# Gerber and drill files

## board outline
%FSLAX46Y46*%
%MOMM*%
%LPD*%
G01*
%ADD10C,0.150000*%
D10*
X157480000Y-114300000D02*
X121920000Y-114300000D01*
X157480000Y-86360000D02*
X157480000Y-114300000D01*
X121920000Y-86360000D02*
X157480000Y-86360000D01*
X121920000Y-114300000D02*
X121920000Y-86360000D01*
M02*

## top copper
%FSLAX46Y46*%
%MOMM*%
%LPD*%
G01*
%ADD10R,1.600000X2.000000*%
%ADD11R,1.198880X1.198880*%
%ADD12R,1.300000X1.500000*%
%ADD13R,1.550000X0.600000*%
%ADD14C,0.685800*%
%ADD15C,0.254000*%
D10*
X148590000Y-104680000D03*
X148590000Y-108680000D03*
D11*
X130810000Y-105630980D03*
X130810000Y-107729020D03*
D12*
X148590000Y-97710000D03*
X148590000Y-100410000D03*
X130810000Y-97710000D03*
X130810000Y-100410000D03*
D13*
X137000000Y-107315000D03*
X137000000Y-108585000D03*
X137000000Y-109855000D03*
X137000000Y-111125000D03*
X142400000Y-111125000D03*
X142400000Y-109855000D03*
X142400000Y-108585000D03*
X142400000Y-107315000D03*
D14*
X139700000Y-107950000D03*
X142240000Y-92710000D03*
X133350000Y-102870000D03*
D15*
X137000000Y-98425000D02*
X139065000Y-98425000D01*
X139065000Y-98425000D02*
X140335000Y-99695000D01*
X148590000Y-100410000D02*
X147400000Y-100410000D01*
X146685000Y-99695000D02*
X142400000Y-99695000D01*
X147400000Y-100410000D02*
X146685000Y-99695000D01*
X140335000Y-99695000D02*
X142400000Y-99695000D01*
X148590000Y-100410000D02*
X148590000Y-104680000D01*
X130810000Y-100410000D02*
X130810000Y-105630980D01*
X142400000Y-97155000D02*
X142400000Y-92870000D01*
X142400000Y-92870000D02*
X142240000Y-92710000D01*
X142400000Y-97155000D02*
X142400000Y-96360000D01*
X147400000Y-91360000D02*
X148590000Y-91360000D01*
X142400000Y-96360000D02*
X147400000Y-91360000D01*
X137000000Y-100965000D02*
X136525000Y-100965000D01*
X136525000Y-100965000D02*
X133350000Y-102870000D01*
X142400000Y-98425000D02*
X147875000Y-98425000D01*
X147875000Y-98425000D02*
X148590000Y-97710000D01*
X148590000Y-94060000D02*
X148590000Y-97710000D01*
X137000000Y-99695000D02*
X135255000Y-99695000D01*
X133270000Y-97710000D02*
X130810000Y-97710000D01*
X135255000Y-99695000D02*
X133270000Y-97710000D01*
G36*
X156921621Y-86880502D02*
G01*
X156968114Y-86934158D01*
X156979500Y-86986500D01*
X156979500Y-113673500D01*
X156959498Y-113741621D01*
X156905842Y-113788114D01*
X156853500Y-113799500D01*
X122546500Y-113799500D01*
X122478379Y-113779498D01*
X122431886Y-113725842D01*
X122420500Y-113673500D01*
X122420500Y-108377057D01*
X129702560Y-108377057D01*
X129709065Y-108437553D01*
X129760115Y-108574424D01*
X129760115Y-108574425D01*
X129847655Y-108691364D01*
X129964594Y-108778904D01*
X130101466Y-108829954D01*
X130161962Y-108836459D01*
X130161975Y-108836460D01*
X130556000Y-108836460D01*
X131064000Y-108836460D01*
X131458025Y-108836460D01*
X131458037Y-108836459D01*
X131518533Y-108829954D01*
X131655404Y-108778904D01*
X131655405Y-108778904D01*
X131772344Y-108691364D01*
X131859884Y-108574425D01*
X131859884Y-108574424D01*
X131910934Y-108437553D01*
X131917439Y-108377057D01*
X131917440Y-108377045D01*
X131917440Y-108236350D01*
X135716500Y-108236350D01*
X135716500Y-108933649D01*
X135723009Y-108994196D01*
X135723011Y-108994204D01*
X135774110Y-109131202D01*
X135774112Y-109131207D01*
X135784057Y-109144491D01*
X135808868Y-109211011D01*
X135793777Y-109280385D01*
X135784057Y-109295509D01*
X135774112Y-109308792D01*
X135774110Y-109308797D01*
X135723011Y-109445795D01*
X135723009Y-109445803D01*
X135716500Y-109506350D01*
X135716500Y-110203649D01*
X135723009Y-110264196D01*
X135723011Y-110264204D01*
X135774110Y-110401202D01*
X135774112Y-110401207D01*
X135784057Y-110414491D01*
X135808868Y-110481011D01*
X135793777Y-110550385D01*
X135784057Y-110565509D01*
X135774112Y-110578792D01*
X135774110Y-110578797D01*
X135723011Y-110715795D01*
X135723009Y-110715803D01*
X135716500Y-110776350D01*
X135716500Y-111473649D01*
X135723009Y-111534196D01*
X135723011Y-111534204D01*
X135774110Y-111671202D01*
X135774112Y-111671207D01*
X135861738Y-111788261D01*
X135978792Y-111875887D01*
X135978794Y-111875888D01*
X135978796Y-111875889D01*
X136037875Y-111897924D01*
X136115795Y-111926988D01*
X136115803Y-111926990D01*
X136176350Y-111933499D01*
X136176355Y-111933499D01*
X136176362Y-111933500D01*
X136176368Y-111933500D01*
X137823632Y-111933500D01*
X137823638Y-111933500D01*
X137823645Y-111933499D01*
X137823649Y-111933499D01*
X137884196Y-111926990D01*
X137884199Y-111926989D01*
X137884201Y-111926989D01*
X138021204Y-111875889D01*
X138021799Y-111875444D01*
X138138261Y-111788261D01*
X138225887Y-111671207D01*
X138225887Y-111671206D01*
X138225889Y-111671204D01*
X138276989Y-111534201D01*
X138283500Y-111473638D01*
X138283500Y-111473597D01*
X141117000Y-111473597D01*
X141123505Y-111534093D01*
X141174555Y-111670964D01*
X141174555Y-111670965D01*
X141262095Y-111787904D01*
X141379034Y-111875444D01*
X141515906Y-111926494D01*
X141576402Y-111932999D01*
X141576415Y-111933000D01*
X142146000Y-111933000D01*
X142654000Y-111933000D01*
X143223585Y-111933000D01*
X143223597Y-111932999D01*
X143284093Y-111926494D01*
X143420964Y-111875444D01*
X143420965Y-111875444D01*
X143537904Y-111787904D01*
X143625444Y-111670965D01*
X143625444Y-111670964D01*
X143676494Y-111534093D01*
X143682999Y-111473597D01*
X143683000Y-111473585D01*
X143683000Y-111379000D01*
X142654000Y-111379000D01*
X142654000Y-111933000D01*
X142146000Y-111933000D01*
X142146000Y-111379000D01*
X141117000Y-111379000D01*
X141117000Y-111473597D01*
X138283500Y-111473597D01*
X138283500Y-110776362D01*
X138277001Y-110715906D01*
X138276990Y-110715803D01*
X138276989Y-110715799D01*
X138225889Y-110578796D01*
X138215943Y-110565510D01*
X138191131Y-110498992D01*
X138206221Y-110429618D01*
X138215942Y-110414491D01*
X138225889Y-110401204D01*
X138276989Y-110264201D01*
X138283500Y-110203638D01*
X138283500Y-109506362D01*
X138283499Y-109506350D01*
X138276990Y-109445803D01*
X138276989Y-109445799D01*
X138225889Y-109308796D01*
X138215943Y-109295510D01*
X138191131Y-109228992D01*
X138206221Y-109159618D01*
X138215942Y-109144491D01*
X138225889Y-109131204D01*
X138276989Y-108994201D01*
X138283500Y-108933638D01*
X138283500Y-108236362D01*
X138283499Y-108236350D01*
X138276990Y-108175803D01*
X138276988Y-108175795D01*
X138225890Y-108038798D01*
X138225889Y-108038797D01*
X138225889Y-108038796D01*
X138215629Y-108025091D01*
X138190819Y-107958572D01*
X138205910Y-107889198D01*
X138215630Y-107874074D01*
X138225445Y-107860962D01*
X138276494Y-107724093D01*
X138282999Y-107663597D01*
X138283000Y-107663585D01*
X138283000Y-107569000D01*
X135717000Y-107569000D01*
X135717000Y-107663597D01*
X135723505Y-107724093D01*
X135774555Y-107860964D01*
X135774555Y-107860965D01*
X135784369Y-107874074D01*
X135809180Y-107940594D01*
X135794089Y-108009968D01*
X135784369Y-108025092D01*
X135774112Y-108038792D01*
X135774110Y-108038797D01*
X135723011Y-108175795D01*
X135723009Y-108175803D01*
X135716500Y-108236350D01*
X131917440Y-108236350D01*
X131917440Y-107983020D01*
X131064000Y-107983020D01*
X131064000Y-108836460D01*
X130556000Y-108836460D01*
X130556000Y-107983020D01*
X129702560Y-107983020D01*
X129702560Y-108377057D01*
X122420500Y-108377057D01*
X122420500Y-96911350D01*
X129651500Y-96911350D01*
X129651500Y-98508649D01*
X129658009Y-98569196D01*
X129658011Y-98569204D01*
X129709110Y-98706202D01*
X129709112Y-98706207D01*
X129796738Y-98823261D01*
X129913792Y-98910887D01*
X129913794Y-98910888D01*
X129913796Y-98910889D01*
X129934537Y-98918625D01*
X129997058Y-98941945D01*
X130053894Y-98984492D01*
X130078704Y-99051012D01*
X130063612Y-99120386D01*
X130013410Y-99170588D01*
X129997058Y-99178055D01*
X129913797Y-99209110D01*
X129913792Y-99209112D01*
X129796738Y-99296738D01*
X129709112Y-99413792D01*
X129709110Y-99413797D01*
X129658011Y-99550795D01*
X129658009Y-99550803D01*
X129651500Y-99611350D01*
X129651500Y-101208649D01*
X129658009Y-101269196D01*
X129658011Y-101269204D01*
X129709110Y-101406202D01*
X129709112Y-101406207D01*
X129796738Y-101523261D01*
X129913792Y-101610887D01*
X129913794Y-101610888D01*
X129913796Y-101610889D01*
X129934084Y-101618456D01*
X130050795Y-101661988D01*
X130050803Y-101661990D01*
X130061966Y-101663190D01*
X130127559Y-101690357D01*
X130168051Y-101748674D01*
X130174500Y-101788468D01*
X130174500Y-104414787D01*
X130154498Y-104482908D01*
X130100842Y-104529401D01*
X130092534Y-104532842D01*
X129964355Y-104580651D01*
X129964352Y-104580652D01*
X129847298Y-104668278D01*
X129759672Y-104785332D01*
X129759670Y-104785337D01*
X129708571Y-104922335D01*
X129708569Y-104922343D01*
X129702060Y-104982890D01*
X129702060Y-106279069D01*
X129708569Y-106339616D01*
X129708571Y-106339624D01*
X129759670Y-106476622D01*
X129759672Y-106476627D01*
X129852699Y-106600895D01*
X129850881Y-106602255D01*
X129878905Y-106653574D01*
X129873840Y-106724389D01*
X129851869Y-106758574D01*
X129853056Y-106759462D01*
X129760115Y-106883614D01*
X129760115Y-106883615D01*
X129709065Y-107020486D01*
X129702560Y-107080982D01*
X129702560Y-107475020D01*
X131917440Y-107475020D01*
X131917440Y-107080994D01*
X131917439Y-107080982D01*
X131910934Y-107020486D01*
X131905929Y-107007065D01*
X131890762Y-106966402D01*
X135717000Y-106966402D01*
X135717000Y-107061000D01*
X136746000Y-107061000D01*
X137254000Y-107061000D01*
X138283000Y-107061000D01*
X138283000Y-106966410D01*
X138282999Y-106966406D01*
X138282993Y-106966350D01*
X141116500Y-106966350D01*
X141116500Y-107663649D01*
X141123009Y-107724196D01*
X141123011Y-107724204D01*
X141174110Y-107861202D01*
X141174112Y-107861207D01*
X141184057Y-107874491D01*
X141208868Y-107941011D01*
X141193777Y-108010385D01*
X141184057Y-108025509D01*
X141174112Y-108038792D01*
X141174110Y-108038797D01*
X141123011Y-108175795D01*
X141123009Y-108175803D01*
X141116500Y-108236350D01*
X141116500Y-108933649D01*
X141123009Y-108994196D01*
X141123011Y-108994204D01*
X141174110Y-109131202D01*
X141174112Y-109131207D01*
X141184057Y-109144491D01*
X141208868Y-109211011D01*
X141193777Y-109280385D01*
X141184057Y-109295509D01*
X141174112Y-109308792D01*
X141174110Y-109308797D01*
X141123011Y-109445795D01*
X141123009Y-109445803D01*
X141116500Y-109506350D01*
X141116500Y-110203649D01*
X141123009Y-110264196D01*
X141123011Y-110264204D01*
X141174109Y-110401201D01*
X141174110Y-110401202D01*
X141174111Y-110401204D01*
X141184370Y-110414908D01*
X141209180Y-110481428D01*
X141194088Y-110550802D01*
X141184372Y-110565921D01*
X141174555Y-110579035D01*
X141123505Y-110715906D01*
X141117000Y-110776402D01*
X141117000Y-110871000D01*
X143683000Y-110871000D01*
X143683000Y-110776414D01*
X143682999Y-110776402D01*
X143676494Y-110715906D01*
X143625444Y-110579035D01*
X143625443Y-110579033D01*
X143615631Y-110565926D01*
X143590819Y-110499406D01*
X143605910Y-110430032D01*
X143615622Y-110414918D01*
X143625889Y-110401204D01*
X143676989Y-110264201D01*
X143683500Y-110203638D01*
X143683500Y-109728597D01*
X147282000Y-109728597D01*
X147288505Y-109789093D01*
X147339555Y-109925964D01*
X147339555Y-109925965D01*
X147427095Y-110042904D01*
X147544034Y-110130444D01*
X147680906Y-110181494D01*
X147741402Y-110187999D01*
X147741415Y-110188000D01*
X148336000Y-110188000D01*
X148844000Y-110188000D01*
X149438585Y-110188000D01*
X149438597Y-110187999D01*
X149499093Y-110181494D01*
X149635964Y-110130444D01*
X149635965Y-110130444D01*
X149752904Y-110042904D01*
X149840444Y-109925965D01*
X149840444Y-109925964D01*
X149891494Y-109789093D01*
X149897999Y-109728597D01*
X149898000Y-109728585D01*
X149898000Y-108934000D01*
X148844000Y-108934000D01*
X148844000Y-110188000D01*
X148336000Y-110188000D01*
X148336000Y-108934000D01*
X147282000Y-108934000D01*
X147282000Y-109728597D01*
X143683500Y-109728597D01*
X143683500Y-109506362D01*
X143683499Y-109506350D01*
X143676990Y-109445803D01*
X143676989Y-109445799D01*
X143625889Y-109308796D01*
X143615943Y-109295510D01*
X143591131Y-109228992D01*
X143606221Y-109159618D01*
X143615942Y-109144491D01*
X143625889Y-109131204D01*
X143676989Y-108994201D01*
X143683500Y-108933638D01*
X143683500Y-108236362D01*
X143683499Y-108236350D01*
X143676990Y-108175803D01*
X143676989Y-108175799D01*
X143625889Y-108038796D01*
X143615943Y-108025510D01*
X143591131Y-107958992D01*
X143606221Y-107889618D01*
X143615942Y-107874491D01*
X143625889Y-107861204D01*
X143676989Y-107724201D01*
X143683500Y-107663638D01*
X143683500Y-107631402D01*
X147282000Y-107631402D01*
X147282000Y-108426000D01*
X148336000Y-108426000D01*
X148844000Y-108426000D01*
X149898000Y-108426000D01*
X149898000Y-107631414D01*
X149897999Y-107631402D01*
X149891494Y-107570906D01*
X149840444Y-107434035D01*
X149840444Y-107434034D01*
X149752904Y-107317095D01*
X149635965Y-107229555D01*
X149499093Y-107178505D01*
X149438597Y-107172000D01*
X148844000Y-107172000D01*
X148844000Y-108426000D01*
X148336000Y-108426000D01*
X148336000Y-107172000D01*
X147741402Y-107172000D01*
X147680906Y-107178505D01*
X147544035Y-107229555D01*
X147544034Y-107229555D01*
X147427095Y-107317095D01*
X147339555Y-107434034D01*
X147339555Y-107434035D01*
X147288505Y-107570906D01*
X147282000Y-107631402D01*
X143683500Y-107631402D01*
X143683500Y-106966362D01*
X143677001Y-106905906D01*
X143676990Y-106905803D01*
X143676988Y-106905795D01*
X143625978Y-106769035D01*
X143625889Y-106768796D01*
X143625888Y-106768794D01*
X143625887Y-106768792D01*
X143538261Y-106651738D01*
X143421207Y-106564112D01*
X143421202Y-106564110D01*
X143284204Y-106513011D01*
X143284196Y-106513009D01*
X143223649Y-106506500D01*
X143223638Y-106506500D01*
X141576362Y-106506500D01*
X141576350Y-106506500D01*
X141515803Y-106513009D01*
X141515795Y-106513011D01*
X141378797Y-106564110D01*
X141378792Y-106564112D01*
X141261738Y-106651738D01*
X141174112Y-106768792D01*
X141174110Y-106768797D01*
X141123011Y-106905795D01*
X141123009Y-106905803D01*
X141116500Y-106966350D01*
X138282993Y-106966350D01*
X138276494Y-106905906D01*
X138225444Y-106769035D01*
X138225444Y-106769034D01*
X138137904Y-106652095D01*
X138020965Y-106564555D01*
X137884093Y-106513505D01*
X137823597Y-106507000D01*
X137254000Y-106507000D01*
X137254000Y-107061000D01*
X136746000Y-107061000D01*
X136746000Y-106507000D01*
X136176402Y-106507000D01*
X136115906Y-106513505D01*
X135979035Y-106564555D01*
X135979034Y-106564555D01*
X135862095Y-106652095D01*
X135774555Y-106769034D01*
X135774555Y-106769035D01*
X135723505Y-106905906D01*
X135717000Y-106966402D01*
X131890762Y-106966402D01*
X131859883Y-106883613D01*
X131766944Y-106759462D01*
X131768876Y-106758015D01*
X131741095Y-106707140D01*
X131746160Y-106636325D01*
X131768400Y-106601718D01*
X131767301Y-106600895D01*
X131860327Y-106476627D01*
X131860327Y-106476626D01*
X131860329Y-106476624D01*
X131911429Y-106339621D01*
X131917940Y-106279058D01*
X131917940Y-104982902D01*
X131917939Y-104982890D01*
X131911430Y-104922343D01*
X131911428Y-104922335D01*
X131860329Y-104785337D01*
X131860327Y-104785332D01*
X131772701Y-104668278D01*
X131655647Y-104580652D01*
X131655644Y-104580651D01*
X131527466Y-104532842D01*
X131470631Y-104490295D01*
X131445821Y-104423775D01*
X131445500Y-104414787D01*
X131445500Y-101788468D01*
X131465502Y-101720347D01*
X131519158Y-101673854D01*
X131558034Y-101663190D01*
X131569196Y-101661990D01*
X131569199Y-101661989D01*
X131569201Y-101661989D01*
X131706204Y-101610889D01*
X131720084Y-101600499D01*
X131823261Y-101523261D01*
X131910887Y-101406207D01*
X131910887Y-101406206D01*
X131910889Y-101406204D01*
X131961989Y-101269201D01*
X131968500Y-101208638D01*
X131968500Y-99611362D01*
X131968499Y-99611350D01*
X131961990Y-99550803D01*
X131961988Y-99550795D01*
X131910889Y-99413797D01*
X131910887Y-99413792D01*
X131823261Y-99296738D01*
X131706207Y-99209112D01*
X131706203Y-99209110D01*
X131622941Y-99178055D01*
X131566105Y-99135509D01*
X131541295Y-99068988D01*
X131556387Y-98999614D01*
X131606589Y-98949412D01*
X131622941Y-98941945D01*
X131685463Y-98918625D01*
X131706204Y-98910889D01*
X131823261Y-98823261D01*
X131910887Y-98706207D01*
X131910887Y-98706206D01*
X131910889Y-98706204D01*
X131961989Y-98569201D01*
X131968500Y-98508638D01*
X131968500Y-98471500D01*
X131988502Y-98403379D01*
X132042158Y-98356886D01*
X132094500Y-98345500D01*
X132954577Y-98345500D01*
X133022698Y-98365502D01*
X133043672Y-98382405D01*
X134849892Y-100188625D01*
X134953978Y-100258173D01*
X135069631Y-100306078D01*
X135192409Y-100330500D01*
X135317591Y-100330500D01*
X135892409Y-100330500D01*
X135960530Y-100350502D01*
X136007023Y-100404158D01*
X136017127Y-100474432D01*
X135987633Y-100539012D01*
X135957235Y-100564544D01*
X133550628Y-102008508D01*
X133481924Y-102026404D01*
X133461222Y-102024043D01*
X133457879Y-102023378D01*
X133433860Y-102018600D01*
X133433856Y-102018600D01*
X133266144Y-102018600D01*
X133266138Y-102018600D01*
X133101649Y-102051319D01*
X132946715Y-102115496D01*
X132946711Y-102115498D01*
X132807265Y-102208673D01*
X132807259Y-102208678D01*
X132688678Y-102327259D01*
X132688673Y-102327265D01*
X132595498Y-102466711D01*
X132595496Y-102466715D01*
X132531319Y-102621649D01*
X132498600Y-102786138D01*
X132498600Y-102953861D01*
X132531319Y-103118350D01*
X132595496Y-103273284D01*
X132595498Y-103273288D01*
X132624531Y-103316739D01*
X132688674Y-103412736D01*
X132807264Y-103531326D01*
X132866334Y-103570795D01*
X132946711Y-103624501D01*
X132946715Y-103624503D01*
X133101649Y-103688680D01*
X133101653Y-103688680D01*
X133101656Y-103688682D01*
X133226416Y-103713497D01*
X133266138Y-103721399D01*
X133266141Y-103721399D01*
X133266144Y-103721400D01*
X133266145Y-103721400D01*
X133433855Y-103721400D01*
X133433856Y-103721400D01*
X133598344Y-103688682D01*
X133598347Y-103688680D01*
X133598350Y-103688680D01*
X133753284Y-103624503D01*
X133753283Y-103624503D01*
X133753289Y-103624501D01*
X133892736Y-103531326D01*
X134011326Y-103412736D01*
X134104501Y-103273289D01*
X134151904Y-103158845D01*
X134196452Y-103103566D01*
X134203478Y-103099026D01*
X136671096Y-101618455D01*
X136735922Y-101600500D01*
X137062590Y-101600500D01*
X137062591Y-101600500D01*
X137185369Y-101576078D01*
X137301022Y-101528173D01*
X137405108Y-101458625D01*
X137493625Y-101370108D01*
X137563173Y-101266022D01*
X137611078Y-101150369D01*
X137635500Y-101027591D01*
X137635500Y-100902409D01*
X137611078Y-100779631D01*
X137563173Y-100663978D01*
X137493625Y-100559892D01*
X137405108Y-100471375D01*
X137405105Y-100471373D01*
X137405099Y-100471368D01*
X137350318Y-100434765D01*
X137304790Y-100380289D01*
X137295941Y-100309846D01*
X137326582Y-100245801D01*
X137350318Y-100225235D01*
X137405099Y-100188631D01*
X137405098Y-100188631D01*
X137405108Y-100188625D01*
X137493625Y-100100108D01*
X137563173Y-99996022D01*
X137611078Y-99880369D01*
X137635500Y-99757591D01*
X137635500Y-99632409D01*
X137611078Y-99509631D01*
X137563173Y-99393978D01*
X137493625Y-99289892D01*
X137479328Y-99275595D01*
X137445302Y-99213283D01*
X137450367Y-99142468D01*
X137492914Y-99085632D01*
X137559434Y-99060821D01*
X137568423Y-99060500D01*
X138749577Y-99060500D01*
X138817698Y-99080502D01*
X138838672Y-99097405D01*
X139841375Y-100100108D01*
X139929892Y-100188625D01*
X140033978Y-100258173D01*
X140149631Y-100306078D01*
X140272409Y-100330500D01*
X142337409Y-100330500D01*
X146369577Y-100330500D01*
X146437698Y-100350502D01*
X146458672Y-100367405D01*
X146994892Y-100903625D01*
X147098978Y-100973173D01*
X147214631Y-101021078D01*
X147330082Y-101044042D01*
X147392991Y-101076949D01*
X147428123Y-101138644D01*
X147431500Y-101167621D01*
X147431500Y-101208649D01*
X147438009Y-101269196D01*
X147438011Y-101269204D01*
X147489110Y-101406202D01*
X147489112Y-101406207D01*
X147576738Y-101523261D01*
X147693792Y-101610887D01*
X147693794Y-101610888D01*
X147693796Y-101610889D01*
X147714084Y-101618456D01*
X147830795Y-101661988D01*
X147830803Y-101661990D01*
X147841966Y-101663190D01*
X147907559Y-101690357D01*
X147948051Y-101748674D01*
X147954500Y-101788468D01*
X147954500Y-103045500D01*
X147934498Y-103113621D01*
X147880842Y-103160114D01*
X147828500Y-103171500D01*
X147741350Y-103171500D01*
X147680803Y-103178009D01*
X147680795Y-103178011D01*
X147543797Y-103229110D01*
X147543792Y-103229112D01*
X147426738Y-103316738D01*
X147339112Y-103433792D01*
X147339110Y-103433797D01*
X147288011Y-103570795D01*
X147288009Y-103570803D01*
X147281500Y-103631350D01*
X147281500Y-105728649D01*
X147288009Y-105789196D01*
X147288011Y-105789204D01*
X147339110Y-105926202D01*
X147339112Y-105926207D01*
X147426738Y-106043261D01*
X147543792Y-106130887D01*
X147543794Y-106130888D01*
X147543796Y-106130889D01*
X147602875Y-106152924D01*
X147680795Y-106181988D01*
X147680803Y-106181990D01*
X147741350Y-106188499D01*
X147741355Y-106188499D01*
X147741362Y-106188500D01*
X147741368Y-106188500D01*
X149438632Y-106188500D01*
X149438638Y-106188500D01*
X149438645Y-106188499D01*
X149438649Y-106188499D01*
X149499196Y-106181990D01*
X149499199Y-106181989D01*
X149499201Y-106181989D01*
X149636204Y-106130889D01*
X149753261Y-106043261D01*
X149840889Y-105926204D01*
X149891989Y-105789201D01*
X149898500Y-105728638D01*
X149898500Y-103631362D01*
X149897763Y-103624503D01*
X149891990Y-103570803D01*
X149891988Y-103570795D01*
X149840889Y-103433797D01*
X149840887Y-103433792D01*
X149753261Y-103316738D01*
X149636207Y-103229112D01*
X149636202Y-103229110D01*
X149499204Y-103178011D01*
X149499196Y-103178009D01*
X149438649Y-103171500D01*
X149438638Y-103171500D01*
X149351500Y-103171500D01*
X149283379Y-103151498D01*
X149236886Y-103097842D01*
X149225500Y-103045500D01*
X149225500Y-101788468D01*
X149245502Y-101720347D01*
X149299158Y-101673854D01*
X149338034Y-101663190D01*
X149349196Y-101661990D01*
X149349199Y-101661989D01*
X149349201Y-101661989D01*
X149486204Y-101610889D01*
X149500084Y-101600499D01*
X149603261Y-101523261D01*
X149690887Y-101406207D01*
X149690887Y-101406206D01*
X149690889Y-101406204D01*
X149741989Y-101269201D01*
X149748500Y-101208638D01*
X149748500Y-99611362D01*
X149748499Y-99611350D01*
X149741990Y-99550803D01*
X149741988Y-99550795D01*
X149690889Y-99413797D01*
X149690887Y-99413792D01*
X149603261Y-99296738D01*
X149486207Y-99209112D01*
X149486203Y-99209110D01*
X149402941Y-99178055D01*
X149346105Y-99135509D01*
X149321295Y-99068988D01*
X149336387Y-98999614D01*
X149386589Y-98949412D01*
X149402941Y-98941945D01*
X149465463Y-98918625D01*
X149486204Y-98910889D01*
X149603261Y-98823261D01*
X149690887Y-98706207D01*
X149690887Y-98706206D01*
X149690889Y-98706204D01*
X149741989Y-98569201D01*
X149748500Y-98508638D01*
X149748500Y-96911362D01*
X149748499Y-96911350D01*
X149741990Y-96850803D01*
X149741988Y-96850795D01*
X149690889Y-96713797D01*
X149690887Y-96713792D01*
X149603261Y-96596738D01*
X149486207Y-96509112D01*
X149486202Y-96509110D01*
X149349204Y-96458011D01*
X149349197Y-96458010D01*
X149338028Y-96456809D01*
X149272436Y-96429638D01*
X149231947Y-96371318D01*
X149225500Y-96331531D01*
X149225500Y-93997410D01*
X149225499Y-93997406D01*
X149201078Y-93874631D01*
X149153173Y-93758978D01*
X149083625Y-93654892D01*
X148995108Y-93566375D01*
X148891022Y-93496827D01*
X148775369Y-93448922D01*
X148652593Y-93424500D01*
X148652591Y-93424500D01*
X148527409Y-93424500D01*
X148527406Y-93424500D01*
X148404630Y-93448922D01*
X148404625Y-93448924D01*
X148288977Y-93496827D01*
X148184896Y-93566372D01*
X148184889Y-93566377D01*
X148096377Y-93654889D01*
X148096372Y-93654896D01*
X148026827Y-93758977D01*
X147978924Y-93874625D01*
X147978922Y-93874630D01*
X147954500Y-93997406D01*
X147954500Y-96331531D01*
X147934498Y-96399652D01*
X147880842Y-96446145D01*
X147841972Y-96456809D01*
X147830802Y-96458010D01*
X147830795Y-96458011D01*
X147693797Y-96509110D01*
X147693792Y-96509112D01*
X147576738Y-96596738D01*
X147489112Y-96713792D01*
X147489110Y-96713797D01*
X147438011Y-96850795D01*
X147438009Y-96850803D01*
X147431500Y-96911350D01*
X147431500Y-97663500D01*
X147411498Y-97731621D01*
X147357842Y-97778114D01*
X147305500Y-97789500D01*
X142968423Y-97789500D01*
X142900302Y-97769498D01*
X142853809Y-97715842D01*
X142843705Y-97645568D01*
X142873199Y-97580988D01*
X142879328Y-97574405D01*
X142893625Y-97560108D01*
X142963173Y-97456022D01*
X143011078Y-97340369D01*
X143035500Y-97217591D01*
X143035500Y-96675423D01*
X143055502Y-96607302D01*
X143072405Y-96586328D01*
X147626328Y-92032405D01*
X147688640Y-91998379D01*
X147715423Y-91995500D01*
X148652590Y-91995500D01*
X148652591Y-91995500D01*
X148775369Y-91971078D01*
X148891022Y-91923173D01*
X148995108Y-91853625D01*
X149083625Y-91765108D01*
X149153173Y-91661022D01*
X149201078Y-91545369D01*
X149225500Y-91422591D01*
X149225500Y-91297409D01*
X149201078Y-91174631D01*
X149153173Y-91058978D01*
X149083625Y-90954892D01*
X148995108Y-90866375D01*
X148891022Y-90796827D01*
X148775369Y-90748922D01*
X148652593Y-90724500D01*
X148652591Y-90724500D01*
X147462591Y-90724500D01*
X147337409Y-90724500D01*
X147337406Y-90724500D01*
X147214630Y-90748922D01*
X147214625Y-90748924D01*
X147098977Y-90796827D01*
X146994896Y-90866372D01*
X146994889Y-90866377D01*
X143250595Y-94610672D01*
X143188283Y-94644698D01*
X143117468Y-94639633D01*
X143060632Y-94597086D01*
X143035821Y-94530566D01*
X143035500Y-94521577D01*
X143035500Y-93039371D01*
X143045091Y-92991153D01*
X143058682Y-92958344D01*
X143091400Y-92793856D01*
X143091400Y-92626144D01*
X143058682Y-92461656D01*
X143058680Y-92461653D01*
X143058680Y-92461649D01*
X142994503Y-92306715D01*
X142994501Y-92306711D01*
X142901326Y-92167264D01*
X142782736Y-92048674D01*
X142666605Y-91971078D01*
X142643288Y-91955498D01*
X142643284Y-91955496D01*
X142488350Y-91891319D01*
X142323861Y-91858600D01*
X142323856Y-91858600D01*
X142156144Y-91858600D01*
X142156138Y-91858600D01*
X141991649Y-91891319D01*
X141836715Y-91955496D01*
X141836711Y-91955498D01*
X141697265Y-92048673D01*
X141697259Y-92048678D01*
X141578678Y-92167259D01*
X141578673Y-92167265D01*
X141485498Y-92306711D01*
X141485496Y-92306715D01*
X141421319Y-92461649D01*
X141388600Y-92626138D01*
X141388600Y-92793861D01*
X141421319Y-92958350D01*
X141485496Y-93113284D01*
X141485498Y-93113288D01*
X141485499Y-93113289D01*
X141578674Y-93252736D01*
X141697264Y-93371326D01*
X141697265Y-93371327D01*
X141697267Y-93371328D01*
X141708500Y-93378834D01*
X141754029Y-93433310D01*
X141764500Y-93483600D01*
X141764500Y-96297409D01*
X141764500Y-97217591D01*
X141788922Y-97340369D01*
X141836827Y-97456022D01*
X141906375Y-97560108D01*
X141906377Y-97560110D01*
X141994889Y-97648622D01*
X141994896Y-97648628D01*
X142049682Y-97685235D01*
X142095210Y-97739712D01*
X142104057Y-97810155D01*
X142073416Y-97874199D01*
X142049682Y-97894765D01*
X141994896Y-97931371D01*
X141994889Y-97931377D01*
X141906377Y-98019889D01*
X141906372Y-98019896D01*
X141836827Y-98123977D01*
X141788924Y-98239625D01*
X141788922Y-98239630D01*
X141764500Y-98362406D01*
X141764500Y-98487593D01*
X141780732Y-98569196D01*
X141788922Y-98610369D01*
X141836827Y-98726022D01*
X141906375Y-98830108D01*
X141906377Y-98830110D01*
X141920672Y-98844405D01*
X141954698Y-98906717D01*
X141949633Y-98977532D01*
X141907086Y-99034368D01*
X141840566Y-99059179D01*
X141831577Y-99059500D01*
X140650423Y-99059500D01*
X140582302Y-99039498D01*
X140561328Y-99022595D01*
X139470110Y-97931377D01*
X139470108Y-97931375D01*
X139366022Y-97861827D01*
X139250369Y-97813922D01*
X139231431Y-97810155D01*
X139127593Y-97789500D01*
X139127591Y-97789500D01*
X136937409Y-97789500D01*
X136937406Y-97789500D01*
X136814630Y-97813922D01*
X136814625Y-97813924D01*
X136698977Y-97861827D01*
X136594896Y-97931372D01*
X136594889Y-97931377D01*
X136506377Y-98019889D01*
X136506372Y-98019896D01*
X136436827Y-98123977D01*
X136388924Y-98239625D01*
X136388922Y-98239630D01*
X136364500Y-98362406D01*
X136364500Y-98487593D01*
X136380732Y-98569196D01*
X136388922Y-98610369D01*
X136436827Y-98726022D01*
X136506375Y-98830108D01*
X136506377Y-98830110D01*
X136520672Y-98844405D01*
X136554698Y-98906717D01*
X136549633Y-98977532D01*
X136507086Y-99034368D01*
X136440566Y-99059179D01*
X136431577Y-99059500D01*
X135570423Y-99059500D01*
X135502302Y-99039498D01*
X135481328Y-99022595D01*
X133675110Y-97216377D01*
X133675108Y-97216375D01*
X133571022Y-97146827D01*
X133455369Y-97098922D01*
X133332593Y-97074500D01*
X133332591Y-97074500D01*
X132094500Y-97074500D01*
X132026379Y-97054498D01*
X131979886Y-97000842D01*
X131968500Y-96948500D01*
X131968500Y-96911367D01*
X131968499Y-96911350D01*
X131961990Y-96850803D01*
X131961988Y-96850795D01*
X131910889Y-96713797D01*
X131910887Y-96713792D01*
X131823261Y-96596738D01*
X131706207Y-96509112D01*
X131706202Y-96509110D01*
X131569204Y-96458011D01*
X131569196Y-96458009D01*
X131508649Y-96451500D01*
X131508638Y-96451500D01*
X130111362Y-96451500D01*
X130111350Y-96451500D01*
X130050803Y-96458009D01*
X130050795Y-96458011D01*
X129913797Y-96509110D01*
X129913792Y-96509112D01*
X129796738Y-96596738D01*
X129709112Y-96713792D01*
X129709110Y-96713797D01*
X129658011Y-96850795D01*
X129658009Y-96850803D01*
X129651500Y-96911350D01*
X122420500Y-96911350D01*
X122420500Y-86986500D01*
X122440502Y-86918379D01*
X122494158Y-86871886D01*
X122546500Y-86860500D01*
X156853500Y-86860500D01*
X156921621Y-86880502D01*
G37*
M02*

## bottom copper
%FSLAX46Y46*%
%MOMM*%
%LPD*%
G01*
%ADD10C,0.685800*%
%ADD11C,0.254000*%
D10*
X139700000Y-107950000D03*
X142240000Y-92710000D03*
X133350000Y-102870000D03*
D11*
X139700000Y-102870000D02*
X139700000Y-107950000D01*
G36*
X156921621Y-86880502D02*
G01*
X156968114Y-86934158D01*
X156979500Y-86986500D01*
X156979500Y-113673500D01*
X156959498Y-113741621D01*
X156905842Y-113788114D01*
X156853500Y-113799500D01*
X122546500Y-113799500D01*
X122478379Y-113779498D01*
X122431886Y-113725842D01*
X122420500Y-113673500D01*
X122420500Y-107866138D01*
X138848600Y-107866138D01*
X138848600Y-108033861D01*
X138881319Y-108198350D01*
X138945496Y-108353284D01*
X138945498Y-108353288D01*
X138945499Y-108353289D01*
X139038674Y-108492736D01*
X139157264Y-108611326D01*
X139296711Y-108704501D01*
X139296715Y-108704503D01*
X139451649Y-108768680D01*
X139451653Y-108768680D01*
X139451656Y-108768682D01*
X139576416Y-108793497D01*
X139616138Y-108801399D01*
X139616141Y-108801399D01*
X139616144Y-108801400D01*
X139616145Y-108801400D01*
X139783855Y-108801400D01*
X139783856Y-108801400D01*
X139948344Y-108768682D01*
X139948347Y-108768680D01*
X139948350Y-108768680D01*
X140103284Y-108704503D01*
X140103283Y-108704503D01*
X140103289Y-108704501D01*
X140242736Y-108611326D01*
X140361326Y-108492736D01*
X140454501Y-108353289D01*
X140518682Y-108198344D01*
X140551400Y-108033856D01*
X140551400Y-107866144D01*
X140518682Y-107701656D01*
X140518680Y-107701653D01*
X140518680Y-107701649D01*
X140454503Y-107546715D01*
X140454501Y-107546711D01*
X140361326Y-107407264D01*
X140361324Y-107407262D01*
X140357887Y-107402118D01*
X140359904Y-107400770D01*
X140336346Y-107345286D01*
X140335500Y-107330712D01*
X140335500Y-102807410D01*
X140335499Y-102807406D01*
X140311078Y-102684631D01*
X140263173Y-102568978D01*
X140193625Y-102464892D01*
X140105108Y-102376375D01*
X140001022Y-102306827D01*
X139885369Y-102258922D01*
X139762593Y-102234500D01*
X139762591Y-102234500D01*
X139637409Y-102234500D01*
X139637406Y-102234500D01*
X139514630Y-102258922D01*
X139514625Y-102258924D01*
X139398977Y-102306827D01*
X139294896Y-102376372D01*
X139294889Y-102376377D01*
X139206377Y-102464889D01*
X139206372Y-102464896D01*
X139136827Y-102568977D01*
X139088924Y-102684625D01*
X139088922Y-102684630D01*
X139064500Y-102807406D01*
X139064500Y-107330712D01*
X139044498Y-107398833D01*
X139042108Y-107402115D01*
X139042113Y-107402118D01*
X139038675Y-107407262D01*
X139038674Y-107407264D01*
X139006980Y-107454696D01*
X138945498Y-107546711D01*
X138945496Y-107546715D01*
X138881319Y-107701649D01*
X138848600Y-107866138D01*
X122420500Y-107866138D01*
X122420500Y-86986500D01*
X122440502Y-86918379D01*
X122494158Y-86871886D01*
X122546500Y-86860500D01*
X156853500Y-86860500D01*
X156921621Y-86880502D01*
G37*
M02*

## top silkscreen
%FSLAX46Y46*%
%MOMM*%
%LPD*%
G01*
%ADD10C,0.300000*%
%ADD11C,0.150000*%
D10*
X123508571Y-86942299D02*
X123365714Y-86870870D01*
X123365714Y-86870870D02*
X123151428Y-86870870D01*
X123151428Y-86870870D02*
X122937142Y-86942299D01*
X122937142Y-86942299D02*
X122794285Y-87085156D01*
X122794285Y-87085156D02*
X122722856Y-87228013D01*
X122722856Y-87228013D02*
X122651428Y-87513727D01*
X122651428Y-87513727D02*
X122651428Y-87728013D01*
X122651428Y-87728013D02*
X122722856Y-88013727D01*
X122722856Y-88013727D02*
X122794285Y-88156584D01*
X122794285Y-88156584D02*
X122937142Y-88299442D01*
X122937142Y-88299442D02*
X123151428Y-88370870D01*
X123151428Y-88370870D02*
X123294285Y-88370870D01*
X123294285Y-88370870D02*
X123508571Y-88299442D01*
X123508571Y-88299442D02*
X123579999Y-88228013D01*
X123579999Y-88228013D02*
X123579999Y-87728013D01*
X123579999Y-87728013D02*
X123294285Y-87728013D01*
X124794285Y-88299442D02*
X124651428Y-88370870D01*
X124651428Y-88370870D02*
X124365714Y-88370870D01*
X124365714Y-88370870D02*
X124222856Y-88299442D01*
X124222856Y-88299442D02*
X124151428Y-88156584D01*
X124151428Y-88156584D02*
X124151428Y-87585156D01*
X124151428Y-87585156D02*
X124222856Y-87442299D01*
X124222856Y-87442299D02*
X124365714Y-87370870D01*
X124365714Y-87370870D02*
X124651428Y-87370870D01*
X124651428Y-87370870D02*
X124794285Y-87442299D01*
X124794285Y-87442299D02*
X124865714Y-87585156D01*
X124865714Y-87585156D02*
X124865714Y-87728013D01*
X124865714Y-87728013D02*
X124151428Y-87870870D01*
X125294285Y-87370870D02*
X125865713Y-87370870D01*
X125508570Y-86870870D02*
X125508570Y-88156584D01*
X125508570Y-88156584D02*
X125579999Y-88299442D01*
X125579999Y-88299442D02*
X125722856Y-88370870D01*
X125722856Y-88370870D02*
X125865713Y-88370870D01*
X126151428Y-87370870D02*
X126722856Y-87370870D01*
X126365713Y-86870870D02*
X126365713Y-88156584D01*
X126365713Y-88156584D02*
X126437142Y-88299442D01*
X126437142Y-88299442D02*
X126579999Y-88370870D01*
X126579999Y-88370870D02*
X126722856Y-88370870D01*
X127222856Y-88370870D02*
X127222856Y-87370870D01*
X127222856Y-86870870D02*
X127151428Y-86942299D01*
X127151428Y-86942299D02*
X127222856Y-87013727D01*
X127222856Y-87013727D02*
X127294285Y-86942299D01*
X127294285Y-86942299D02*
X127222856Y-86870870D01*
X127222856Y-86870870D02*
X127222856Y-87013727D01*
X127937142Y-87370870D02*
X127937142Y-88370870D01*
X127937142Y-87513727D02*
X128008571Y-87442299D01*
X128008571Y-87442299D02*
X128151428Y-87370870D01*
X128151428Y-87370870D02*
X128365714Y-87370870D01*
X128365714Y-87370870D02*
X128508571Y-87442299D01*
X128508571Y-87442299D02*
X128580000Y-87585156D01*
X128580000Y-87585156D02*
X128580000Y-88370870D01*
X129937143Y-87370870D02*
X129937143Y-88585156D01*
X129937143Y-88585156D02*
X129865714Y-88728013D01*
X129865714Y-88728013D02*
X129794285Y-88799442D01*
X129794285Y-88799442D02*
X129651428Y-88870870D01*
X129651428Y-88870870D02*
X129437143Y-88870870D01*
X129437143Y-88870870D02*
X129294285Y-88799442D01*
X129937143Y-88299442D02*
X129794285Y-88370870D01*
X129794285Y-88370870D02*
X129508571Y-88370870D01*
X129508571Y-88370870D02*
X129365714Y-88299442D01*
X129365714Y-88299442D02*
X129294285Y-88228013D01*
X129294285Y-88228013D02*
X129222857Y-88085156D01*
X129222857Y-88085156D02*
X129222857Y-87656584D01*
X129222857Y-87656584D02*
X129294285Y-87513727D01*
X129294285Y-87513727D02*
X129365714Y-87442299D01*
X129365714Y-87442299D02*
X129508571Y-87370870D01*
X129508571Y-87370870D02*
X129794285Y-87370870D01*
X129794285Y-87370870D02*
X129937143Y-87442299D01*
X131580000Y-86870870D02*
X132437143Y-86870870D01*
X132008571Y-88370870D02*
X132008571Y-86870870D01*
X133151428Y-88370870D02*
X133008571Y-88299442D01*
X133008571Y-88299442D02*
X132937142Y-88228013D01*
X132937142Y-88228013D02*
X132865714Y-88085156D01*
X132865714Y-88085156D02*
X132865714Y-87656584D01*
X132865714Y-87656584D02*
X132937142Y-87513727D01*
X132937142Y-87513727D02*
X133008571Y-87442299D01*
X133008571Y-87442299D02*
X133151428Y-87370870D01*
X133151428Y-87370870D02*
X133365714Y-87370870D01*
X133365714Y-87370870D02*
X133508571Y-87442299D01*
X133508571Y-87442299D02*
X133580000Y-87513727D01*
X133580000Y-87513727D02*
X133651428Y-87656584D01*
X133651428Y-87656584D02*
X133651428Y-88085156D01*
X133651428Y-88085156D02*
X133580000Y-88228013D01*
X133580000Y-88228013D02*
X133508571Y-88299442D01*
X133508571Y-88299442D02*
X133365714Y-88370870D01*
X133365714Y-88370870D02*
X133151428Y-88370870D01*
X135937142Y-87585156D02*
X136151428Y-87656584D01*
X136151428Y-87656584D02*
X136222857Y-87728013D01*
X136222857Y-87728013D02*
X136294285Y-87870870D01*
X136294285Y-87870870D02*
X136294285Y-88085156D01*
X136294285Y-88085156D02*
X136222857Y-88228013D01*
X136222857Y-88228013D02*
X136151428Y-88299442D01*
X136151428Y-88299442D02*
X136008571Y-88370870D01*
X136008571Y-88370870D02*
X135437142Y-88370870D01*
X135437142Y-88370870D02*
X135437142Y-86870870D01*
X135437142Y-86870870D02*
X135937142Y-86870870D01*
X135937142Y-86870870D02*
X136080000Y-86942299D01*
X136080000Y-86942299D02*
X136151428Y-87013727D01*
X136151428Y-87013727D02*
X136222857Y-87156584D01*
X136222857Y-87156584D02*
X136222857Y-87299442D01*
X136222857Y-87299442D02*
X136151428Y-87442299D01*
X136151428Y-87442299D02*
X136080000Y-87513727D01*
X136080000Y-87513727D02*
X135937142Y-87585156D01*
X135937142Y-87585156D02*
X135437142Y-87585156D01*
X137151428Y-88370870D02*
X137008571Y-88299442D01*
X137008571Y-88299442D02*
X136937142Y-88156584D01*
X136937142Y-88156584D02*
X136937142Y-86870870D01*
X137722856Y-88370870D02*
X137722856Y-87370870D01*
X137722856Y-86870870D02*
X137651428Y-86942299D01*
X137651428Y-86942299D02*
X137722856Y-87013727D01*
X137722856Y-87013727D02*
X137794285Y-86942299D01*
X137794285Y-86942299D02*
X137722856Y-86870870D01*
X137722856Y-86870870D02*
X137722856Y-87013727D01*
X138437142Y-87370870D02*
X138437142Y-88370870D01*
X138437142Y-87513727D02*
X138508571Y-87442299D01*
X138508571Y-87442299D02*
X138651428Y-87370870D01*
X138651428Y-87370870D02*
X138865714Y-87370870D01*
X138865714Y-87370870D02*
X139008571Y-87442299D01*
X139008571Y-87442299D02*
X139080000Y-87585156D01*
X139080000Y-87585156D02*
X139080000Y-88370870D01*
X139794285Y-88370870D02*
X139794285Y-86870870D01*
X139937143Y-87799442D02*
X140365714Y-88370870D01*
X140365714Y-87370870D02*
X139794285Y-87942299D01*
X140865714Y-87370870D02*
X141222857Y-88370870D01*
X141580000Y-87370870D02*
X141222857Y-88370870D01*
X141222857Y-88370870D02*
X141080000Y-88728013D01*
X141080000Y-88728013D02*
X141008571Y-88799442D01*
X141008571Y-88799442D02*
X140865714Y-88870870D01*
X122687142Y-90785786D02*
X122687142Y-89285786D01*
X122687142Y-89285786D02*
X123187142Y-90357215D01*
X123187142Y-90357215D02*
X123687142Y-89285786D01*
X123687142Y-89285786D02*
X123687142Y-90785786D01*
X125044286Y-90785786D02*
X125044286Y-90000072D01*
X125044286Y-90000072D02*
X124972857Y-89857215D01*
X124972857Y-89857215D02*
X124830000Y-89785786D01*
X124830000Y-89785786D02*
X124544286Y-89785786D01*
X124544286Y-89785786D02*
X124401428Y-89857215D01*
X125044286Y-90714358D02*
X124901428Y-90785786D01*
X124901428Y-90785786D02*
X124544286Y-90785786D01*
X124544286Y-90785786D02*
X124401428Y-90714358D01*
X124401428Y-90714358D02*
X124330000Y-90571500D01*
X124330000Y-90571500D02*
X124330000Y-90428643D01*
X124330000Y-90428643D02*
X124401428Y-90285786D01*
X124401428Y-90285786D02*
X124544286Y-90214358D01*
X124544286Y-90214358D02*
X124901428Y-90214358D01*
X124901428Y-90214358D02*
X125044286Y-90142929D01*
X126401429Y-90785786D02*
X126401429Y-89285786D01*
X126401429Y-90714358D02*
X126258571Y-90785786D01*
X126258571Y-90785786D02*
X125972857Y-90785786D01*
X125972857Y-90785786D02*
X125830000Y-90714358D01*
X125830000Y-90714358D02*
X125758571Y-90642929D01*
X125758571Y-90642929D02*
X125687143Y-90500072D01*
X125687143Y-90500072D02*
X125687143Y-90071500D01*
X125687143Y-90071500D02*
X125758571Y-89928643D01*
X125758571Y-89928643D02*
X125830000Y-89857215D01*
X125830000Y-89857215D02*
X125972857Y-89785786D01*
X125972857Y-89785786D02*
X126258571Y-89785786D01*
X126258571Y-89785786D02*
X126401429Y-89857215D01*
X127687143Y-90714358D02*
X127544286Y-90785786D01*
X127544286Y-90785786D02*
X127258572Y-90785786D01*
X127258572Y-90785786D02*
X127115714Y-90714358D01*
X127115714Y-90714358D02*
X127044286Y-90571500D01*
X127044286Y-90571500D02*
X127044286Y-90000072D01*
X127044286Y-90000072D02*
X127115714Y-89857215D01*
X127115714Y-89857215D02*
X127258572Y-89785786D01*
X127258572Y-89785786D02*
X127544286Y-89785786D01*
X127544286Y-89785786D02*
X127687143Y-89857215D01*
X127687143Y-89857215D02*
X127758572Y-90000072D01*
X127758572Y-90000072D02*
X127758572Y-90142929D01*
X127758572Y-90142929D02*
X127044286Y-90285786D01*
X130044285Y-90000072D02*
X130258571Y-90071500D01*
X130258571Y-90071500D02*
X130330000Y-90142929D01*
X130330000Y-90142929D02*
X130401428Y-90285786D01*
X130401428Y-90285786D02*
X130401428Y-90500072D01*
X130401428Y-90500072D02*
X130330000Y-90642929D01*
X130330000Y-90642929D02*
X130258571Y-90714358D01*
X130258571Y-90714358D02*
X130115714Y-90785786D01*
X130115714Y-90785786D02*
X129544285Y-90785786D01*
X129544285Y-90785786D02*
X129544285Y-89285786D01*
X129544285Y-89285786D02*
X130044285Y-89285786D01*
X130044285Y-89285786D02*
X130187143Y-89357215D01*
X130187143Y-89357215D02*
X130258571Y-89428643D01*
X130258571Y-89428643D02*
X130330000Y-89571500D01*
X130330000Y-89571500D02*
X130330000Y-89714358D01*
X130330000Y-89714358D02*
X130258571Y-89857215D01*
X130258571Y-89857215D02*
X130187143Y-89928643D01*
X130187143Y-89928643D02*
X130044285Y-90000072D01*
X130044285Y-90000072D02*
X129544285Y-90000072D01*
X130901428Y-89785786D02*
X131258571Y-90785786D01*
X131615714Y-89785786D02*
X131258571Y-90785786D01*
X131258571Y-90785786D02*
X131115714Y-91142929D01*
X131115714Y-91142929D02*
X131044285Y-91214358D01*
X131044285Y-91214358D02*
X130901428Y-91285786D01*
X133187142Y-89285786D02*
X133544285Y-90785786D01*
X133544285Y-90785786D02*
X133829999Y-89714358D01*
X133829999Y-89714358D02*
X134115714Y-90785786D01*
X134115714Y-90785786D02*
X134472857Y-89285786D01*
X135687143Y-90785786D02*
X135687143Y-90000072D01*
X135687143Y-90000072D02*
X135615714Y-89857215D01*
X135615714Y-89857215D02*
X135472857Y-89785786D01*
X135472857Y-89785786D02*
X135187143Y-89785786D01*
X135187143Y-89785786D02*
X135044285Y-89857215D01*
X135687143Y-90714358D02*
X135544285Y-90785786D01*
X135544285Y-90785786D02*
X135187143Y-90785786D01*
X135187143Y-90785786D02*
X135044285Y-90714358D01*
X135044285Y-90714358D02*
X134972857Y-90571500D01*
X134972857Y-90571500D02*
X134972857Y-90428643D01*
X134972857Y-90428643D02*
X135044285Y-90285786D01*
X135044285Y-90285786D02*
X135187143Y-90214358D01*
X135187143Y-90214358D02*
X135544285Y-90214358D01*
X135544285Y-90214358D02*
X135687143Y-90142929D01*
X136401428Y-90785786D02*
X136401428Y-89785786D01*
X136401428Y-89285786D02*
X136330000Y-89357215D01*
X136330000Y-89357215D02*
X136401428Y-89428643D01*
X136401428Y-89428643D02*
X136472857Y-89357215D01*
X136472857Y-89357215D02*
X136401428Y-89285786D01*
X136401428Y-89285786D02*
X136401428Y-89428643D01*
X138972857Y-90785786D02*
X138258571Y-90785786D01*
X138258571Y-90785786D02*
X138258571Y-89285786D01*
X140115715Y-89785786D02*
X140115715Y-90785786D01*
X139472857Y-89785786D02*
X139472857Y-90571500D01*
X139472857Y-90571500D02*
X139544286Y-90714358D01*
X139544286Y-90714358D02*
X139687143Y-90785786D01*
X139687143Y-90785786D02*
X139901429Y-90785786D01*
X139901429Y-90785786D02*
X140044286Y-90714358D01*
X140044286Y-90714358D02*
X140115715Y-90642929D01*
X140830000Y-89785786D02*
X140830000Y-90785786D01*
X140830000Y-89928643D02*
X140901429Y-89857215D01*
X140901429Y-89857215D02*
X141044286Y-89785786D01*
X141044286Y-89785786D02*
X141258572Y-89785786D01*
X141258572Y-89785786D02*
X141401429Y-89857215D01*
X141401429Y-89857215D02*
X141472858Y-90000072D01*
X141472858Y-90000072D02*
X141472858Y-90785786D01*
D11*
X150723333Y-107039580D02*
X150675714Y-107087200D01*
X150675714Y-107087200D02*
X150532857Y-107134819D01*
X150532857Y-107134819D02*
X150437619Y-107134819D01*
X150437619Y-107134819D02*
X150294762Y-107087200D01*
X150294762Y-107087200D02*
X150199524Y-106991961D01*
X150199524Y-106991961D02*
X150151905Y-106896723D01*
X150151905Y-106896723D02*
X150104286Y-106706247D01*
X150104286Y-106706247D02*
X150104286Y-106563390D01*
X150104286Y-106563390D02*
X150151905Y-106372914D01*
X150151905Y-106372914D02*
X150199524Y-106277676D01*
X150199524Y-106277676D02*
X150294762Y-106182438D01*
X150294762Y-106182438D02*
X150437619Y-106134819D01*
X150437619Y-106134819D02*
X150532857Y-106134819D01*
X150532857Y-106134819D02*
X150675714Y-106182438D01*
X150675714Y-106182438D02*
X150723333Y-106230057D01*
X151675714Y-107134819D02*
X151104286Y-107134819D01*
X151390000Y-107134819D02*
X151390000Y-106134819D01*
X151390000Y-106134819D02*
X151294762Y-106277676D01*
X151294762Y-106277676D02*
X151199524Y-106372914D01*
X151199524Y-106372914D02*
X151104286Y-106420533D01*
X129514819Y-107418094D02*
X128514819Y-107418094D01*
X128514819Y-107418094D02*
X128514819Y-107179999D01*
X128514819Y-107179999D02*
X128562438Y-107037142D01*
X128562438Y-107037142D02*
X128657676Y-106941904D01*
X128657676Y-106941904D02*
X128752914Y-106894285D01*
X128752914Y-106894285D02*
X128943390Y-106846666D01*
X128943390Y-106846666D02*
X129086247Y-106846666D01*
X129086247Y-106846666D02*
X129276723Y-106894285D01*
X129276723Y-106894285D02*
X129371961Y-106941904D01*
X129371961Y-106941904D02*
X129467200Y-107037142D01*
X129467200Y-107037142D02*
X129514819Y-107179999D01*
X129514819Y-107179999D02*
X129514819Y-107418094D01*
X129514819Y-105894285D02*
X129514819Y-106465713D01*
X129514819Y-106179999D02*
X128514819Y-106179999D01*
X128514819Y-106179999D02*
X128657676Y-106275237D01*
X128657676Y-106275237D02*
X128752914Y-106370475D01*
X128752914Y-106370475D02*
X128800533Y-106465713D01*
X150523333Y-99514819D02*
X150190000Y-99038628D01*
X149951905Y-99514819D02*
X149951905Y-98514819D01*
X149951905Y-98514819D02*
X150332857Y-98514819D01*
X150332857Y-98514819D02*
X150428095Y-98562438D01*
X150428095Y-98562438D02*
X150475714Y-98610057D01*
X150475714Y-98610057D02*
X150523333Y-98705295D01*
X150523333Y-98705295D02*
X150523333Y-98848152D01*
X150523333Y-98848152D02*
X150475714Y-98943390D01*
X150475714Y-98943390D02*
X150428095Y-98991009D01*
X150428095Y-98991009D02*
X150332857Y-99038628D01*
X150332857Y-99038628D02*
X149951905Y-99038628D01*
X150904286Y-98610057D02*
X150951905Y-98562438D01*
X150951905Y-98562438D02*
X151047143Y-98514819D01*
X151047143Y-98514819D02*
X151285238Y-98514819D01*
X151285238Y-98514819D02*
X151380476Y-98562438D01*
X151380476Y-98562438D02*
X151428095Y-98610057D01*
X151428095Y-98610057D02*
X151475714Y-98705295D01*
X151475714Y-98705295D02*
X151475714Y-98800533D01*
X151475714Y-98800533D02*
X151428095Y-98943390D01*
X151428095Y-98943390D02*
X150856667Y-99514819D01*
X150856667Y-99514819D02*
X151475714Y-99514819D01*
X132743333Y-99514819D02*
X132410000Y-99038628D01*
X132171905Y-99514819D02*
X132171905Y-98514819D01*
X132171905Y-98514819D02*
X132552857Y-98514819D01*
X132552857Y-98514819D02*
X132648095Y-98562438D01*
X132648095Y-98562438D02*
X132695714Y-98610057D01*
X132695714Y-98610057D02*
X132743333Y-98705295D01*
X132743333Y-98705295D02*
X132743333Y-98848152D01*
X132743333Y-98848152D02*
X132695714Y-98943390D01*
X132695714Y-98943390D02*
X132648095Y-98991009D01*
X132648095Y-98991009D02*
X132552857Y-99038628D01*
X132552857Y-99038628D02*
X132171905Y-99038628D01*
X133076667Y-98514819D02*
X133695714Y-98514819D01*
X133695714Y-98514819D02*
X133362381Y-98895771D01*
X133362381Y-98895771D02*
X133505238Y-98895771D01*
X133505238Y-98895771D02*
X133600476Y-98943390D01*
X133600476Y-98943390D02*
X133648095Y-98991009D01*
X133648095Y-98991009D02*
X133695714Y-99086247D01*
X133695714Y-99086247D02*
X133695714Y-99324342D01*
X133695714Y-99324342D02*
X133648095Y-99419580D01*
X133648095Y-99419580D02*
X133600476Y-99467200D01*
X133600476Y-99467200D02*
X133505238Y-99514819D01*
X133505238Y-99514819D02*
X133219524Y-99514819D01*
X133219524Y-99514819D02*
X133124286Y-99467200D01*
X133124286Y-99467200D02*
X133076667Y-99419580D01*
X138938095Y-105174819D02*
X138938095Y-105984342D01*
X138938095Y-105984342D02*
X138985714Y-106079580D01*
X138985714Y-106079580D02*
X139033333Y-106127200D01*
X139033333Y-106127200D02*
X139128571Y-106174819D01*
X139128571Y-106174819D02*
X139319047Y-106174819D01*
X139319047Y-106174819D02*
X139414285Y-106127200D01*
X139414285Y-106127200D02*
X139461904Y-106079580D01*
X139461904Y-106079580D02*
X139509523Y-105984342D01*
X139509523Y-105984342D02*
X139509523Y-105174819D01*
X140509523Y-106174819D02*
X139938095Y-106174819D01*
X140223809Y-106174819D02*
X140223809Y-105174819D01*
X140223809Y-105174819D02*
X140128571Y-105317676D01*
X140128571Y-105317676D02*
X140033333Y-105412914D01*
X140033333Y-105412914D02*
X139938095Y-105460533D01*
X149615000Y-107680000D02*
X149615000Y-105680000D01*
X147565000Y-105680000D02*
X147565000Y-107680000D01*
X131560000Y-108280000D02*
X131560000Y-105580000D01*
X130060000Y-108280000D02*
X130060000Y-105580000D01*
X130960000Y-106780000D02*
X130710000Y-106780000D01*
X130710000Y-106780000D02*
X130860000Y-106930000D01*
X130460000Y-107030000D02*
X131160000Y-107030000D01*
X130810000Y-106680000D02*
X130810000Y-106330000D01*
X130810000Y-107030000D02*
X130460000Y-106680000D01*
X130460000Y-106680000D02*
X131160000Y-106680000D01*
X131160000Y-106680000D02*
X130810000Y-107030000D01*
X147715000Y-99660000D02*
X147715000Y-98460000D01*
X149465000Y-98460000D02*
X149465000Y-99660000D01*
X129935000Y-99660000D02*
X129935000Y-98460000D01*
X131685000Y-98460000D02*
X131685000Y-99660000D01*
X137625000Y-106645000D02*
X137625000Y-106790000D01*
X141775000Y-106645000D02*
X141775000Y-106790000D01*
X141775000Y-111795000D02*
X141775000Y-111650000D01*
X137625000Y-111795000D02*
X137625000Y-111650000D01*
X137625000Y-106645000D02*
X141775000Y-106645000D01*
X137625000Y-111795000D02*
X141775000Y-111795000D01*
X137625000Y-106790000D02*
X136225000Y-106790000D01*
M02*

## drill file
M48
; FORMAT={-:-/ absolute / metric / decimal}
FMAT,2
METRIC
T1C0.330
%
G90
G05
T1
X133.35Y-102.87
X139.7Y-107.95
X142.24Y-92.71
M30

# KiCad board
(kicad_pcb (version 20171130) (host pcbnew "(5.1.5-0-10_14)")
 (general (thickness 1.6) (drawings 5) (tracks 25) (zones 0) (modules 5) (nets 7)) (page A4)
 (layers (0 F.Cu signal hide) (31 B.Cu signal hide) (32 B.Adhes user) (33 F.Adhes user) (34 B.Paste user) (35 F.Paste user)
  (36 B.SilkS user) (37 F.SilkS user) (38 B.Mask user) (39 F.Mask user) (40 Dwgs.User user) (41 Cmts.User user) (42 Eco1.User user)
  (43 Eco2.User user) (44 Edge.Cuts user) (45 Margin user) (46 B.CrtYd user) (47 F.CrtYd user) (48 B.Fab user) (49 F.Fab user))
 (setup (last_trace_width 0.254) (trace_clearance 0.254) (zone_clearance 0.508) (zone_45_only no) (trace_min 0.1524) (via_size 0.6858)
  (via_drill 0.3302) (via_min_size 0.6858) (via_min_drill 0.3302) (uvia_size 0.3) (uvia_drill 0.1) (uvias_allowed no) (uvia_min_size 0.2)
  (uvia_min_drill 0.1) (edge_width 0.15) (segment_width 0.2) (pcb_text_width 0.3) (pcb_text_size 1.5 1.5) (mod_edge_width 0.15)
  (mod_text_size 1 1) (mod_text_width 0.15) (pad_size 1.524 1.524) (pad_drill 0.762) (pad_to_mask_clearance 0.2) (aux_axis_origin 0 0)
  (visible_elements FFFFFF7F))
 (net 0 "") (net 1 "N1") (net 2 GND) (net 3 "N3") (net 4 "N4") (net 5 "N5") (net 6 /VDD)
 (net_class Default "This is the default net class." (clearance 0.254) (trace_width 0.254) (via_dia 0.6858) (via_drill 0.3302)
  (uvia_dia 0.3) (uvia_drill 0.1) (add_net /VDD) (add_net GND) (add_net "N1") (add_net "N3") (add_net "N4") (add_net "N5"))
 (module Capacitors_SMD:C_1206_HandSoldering (layer F.Cu) (at 148.59 106.68 270)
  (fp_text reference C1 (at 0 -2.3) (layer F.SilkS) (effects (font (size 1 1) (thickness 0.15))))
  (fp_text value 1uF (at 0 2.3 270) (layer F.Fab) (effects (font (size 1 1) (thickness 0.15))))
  (fp_line (start 1 -1.025) (end -1 -1.025) (layer F.SilkS) (width 0.15))
  (fp_line (start -1 1.025) (end 1 1.025) (layer F.SilkS) (width 0.15))
  (pad 1 smd rect (at -2 0 270) (size 2 1.6) (layers F.Cu F.Paste F.Mask) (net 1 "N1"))
  (pad 2 smd rect (at 2 0 270) (size 2 1.6) (layers F.Cu F.Paste F.Mask) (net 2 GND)))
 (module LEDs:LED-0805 (layer F.Cu) (at 130.81 106.68 90)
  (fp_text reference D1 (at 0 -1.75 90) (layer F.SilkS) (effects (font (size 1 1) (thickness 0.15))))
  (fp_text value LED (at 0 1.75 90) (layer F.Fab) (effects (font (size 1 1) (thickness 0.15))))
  (fp_line (start -1.6 0.75) (end 1.1 0.75) (layer F.SilkS) (width 0.15))
  (fp_line (start -1.6 -0.75) (end 1.1 -0.75) (layer F.SilkS) (width 0.15))
  (fp_line (start -0.1 0.15) (end -0.1 -0.1) (layer F.SilkS) (width 0.15))
  (fp_line (start -0.1 -0.1) (end -0.25 0.05) (layer F.SilkS) (width 0.15))
  (fp_line (start -0.35 -0.35) (end -0.35 0.35) (layer F.SilkS) (width 0.15))
  (fp_line (start 0 0) (end 0.35 0) (layer F.SilkS) (width 0.15))
  (fp_line (start -0.35 0) (end 0 -0.35) (layer F.SilkS) (width 0.15))
  (fp_line (start 0 -0.35) (end 0 0.35) (layer F.SilkS) (width 0.15))
  (fp_line (start 0 0.35) (end -0.35 0) (layer F.SilkS) (width 0.15))
  (pad 2 smd rect (at 1.04902 0 270) (size 1.19888 1.19888) (layers F.Cu F.Paste F.Mask) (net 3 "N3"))
  (pad 1 smd rect (at -1.04902 0 270) (size 1.19888 1.19888) (layers F.Cu F.Paste F.Mask) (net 2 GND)))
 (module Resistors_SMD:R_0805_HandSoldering (layer F.Cu) (at 148.59 99.06 270)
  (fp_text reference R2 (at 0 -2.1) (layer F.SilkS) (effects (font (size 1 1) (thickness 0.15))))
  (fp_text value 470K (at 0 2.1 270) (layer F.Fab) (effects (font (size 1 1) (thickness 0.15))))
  (fp_line (start 0.6 0.875) (end -0.6 0.875) (layer F.SilkS) (width 0.15))
  (fp_line (start -0.6 -0.875) (end 0.6 -0.875) (layer F.SilkS) (width 0.15))
  (pad 1 smd rect (at -1.35 0 270) (size 1.5 1.3) (layers F.Cu F.Paste F.Mask) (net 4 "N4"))
  (pad 2 smd rect (at 1.35 0 270) (size 1.5 1.3) (layers F.Cu F.Paste F.Mask) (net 1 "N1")))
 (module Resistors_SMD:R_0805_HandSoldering (layer F.Cu) (at 130.81 99.06 270)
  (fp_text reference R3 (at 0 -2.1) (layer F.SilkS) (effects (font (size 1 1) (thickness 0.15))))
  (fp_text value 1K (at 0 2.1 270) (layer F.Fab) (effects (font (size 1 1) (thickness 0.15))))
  (fp_line (start 0.6 0.875) (end -0.6 0.875) (layer F.SilkS) (width 0.15))
  (fp_line (start -0.6 -0.875) (end 0.6 -0.875) (layer F.SilkS) (width 0.15))
  (pad 1 smd rect (at -1.35 0 270) (size 1.5 1.3) (layers F.Cu F.Paste F.Mask) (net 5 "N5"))
  (pad 2 smd rect (at 1.35 0 270) (size 1.5 1.3) (layers F.Cu F.Paste F.Mask) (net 3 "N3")))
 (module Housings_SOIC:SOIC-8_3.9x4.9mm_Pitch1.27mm (layer F.Cu) (at 139.7 109.22)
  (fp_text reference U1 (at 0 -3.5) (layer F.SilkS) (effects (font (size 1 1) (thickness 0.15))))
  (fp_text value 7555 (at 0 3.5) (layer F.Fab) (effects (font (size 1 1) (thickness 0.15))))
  (fp_line (start -2.075 -2.575) (end -2.075 -2.43) (layer F.SilkS) (width 0.15))
  (fp_line (start 2.075 -2.575) (end 2.075 -2.43) (layer F.SilkS) (width 0.15))
  (fp_line (start 2.075 2.575) (end 2.075 2.43) (layer F.SilkS) (width 0.15))
  (fp_line (start -2.075 2.575) (end -2.075 2.43) (layer F.SilkS) (width 0.15))
  (fp_line (start -2.075 -2.575) (end 2.075 -2.575) (layer F.SilkS) (width 0.15))
  (fp_line (start -2.075 2.575) (end 2.075 2.575) (layer F.SilkS) (width 0.15))
  (fp_line (start -2.075 -2.43) (end -3.475 -2.43) (layer F.SilkS) (width 0.15))
  (pad 1 smd rect (at -2.7 -1.905) (size 1.55 0.6) (layers F.Cu F.Paste F.Mask) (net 2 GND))
  (pad 2 smd rect (at -2.7 -0.635) (size 1.55 0.6) (layers F.Cu F.Paste F.Mask) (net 1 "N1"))
  (pad 3 smd rect (at -2.7 0.635) (size 1.55 0.6) (layers F.Cu F.Paste F.Mask) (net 5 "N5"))
  (pad 4 smd rect (at -2.7 1.905) (size 1.55 0.6) (layers F.Cu F.Paste F.Mask) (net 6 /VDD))
  (pad 5 smd rect (at 2.7 1.905) (size 1.55 0.6) (layers F.Cu F.Paste F.Mask) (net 2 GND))
  (pad 6 smd rect (at 2.7 0.635) (size 1.55 0.6) (layers F.Cu F.Paste F.Mask) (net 1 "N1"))
  (pad 7 smd rect (at 2.7 -0.635) (size 1.55 0.6) (layers F.Cu F.Paste F.Mask) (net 4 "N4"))
  (pad 8 smd rect (at 2.7 -1.905) (size 1.55 0.6) (layers F.Cu F.Paste F.Mask) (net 6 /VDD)))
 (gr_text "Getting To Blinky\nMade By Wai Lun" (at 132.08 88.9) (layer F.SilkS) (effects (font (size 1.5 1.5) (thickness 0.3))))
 (gr_line (start 157.48 114.3) (end 121.92 114.3) (angle 90) (layer Edge.Cuts) (width 0.15))
 (gr_line (start 157.48 86.36) (end 157.48 114.3) (angle 90) (layer Edge.Cuts) (width 0.15))
 (gr_line (start 121.92 86.36) (end 157.48 86.36) (angle 90) (layer Edge.Cuts) (width 0.15))
 (gr_line (start 121.92 114.3) (end 121.92 86.36) (angle 90) (layer Edge.Cuts) (width 0.15))
 (segment (start 137 98.425) (end 139.065 98.425) (width 0.254) (layer F.Cu) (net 1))
 (segment (start 139.065 98.425) (end 140.335 99.695) (width 0.254) (layer F.Cu) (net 1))
 (segment (start 148.59 100.41) (end 147.4 100.41) (width 0.254) (layer F.Cu) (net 1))
 (segment (start 146.685 99.695) (end 142.4 99.695) (width 0.254) (layer F.Cu) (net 1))
 (segment (start 147.4 100.41) (end 146.685 99.695) (width 0.254) (layer F.Cu) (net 1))
 (segment (start 140.335 99.695) (end 142.4 99.695) (width 0.254) (layer F.Cu) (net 1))
 (segment (start 148.59 100.41) (end 148.59 104.68) (width 0.254) (layer F.Cu) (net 1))
 (segment (start 139.7 102.87) (end 139.7 107.95) (width 0.254) (layer B.Cu) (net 2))
 (via (at 139.7 107.95) (size 0.6858) (drill 0.3302) (layers F.Cu B.Cu) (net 2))
 (segment (start 130.81 100.41) (end 130.81 105.63098) (width 0.254) (layer F.Cu) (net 3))
 (segment (start 142.4 97.155) (end 142.4 92.87) (width 0.254) (layer F.Cu) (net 6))
 (via (at 142.24 92.71) (size 0.6858) (drill 0.3302) (layers F.Cu B.Cu) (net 6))
 (segment (start 142.4 92.87) (end 142.24 92.71) (width 0.254) (layer F.Cu) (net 6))
 (segment (start 142.4 97.155) (end 142.4 96.36) (width 0.254) (layer F.Cu) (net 6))
 (segment (start 147.4 91.36) (end 148.59 91.36) (width 0.254) (layer F.Cu) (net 6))
 (segment (start 142.4 96.36) (end 147.4 91.36) (width 0.254) (layer F.Cu) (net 6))
 (segment (start 137 100.965) (end 136.525 100.965) (width 0.254) (layer F.Cu) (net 6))
 (segment (start 136.525 100.965) (end 133.35 102.87) (width 0.254) (layer F.Cu) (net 6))
 (via (at 133.35 102.87) (size 0.6858) (drill 0.3302) (layers F.Cu B.Cu) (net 6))
 (segment (start 142.4 98.425) (end 147.875 98.425) (width 0.254) (layer F.Cu) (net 4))
 (segment (start 147.875 98.425) (end 148.59 97.71) (width 0.254) (layer F.Cu) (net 4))
 (segment (start 148.59 94.06) (end 148.59 97.71) (width 0.254) (layer F.Cu) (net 4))
 (segment (start 137 99.695) (end 135.255 99.695) (width 0.254) (layer F.Cu) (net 5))
 (segment (start 133.27 97.71) (end 130.81 97.71) (width 0.254) (layer F.Cu) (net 5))
 (segment (start 135.255 99.695) (end 133.27 97.71) (width 0.254) (layer F.Cu) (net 5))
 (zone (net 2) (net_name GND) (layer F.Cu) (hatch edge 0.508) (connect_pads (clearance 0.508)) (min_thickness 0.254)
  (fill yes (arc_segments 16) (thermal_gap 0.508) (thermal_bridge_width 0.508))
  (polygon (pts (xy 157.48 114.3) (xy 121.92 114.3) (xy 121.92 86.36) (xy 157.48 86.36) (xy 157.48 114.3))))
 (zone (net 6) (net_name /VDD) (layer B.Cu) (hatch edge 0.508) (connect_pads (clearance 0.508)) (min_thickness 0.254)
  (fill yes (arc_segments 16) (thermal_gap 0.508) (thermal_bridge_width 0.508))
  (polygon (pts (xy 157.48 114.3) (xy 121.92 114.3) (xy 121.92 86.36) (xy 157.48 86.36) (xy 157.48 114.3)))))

